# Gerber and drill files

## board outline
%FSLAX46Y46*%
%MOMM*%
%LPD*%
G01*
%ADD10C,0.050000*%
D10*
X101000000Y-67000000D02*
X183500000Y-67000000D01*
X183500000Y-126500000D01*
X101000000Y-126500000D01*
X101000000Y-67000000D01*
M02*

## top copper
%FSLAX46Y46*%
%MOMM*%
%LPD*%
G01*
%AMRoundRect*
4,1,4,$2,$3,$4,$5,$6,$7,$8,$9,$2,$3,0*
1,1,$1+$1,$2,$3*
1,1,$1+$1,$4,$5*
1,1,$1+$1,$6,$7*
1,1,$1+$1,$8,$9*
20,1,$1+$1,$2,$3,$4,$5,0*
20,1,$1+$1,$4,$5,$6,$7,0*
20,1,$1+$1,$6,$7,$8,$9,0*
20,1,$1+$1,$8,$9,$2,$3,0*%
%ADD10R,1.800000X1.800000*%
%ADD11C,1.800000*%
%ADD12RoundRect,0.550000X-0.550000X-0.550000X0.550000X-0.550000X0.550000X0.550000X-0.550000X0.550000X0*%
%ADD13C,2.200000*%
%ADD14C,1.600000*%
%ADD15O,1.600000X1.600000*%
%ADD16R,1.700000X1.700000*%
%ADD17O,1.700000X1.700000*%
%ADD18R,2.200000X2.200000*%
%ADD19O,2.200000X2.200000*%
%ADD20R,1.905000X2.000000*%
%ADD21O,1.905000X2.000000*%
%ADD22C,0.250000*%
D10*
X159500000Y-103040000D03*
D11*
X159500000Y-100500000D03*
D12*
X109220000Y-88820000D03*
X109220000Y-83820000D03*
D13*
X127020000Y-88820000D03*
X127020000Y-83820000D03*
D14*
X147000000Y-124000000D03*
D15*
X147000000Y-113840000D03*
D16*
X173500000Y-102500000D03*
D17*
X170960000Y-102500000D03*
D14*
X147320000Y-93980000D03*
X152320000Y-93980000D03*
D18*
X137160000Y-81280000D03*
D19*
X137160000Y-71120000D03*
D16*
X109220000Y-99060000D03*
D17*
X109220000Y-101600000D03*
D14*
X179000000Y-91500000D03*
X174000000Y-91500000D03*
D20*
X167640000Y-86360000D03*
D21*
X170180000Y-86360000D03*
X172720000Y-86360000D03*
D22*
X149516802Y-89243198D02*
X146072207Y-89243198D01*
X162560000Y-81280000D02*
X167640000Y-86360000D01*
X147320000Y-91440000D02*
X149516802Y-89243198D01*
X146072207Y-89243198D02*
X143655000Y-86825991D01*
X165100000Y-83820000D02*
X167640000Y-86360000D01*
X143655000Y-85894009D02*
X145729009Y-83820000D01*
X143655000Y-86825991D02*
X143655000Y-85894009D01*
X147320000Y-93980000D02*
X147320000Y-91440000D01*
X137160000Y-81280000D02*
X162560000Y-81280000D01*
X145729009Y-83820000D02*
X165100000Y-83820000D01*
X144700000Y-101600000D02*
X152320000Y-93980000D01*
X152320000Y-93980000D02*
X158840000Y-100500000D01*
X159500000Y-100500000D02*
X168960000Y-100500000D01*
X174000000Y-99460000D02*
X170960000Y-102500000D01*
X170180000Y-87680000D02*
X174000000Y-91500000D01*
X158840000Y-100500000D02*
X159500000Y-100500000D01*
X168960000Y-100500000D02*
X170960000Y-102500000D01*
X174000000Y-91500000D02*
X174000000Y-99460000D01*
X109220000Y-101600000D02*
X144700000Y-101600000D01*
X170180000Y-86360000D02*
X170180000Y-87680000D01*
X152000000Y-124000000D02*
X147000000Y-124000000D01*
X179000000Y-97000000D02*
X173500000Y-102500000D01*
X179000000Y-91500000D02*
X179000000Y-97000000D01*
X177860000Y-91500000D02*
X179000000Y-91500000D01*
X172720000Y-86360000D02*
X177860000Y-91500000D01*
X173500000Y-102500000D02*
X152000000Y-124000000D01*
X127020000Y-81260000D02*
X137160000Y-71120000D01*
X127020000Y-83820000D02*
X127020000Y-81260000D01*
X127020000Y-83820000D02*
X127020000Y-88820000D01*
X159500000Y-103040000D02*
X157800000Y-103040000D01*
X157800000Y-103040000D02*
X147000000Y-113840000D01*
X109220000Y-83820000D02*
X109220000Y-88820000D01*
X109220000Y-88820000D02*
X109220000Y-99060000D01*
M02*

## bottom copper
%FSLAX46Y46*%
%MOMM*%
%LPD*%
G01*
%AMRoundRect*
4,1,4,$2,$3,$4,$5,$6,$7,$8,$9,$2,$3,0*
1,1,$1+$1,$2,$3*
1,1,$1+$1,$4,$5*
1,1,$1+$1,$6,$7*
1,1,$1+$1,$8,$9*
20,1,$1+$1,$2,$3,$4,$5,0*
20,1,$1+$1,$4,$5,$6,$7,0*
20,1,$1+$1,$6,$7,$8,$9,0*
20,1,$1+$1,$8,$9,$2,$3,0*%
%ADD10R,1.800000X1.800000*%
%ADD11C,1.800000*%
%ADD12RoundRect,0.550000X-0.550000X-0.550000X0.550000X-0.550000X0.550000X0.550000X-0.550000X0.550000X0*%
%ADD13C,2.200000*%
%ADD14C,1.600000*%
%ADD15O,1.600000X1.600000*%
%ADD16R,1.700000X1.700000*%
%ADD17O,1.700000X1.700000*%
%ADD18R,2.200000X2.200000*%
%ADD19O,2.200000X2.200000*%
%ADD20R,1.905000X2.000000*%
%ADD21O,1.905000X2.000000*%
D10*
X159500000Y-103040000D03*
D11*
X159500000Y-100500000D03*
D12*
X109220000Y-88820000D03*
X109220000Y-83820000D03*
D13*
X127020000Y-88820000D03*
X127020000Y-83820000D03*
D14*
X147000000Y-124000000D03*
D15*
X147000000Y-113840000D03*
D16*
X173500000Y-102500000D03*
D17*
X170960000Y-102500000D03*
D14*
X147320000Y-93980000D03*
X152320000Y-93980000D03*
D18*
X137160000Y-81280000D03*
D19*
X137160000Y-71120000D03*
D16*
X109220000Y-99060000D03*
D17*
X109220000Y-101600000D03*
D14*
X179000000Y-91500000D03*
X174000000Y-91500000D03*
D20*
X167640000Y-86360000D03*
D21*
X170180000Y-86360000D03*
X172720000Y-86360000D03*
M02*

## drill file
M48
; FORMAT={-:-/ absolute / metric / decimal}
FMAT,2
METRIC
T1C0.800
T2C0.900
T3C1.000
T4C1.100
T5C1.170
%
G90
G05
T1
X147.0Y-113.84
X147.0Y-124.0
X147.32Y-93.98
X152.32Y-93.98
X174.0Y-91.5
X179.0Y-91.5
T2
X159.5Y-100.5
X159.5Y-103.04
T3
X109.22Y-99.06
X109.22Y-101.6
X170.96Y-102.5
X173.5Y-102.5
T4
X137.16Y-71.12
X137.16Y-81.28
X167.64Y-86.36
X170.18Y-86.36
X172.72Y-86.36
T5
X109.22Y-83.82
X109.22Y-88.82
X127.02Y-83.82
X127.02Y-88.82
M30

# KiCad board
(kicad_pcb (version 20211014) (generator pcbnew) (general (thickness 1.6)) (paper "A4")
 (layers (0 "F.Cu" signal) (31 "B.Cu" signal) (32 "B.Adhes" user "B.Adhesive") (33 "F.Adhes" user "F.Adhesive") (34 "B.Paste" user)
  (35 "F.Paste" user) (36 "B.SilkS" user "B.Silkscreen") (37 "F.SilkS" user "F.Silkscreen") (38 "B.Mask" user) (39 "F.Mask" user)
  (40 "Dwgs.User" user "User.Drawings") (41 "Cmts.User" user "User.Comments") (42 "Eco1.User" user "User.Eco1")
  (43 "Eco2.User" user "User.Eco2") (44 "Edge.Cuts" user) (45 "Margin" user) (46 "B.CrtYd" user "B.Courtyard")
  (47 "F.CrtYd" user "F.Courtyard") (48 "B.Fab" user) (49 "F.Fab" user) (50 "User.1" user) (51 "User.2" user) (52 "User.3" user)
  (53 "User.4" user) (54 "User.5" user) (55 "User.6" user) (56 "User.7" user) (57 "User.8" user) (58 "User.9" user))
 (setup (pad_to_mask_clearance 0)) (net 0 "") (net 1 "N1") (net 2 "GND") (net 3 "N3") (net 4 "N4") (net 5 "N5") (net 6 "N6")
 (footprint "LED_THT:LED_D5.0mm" (layer "F.Cu") (at 159.5 103.04 90)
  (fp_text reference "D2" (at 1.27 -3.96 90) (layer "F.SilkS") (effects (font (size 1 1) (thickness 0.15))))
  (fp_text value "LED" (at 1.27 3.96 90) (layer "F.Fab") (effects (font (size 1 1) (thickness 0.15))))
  (pad "1" thru_hole rect (at 0 0 90) (size 1.8 1.8) (drill 0.9) (layers *.Cu *.Mask) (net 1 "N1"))
  (pad "2" thru_hole circle (at 2.54 0 90) (size 1.8 1.8) (drill 0.9) (layers *.Cu *.Mask) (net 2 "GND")))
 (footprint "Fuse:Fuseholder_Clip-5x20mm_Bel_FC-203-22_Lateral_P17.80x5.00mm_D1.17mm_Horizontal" (layer "F.Cu") (at 109.22 83.82)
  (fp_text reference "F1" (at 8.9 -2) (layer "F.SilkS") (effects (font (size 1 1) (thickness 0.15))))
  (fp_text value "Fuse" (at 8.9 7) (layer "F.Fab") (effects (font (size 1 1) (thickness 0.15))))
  (pad "1" thru_hole roundrect (at 0 5) (size 2.2 2.2) (drill 1.17) (layers *.Cu *.Mask) (roundrect_rratio 0.25) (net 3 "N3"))
  (pad "1" thru_hole roundrect (at 0 0) (size 2.2 2.2) (drill 1.17) (layers *.Cu *.Mask) (roundrect_rratio 0.25) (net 3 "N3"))
  (pad "2" thru_hole circle (at 17.8 5) (size 2.2 2.2) (drill 1.17) (layers *.Cu *.Mask) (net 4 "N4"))
  (pad "2" thru_hole circle (at 17.8 0) (size 2.2 2.2) (drill 1.17) (layers *.Cu *.Mask) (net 4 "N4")))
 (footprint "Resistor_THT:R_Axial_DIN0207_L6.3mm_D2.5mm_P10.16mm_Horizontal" (layer "F.Cu") (at 147 124 90)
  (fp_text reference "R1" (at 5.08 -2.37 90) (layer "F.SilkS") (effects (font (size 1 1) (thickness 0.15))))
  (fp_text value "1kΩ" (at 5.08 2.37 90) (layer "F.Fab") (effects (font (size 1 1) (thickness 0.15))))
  (pad "1" thru_hole circle (at 0 0 90) (size 1.6 1.6) (drill 0.8) (layers *.Cu *.Mask) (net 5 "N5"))
  (pad "2" thru_hole oval (at 10.16 0 90) (size 1.6 1.6) (drill 0.8) (layers *.Cu *.Mask) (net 1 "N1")))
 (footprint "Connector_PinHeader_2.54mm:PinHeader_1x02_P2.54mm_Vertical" (layer "F.Cu") (at 173.5 102.5 -90)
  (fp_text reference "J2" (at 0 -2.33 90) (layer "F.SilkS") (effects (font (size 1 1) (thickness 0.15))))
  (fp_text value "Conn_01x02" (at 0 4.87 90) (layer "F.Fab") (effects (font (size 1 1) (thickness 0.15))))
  (pad "1" thru_hole rect (at 0 0 270) (size 1.7 1.7) (drill 1) (layers *.Cu *.Mask) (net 5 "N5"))
  (pad "2" thru_hole oval (at 0 2.54 270) (size 1.7 1.7) (drill 1) (layers *.Cu *.Mask) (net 2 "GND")))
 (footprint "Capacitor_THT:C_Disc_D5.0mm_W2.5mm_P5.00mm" (layer "F.Cu") (at 147.32 93.98)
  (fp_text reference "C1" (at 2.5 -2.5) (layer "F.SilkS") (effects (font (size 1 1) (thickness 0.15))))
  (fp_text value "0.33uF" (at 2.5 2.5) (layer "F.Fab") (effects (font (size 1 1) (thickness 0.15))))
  (pad "1" thru_hole circle (at 0 0) (size 1.6 1.6) (drill 0.8) (layers *.Cu *.Mask) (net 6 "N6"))
  (pad "2" thru_hole circle (at 5 0) (size 1.6 1.6) (drill 0.8) (layers *.Cu *.Mask) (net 2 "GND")))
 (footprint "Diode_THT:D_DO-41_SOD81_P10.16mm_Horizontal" (layer "F.Cu") (at 137.16 81.28 90)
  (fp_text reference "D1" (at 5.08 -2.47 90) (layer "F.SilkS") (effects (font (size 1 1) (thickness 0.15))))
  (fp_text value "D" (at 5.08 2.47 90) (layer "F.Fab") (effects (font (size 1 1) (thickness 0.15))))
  (pad "1" thru_hole rect (at 0 0 90) (size 2.2 2.2) (drill 1.1) (layers *.Cu *.Mask) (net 6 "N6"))
  (pad "2" thru_hole oval (at 10.16 0 90) (size 2.2 2.2) (drill 1.1) (layers *.Cu *.Mask) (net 4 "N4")))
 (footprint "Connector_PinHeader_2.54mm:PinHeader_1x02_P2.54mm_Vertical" (layer "F.Cu") (at 109.22 99.06)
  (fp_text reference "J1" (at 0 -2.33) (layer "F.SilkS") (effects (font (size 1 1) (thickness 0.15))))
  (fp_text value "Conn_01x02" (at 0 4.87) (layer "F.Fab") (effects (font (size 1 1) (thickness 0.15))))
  (pad "1" thru_hole rect (at 0 0) (size 1.7 1.7) (drill 1) (layers *.Cu *.Mask) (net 3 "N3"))
  (pad "2" thru_hole oval (at 0 2.54) (size 1.7 1.7) (drill 1) (layers *.Cu *.Mask) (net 2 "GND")))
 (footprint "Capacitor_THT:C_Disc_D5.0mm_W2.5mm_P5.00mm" (layer "B.Cu") (at 179 91.5 180)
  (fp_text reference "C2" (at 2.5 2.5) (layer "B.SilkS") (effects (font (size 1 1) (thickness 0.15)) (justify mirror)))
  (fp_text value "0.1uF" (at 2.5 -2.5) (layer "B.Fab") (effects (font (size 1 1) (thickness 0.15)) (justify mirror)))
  (pad "1" thru_hole circle (at 0 0 180) (size 1.6 1.6) (drill 0.8) (layers *.Cu *.Mask) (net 5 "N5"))
  (pad "2" thru_hole circle (at 5 0 180) (size 1.6 1.6) (drill 0.8) (layers *.Cu *.Mask) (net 2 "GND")))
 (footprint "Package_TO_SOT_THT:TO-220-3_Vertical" (layer "B.Cu") (at 167.64 86.36)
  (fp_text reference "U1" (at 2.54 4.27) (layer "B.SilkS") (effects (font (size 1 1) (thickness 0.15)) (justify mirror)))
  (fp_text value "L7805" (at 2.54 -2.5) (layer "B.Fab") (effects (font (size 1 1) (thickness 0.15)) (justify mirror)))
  (pad "1" thru_hole rect (at 0 0) (size 1.905 2) (drill 1.1) (layers *.Cu *.Mask) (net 6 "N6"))
  (pad "2" thru_hole oval (at 2.54 0) (size 1.905 2) (drill 1.1) (layers *.Cu *.Mask) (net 2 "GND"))
  (pad "3" thru_hole oval (at 5.08 0) (size 1.905 2) (drill 1.1) (layers *.Cu *.Mask) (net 5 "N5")))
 (gr_rect (start 101 67) (end 183.5 126.5) (layer "Edge.Cuts") (width 0.05) (fill none))
 (segment (start 149.516802 89.243198) (end 146.072207 89.243198) (width 0.25) (layer "F.Cu") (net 6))
 (segment (start 162.56 81.28) (end 167.64 86.36) (width 0.25) (layer "F.Cu") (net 6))
 (segment (start 147.32 91.44) (end 149.516802 89.243198) (width 0.25) (layer "F.Cu") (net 6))
 (segment (start 146.072207 89.243198) (end 143.655 86.825991) (width 0.25) (layer "F.Cu") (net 6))
 (segment (start 165.1 83.82) (end 167.64 86.36) (width 0.25) (layer "F.Cu") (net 6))
 (segment (start 143.655 85.894009) (end 145.729009 83.82) (width 0.25) (layer "F.Cu") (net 6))
 (segment (start 143.655 86.825991) (end 143.655 85.894009) (width 0.25) (layer "F.Cu") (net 6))
 (segment (start 147.32 93.98) (end 147.32 91.44) (width 0.25) (layer "F.Cu") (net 6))
 (segment (start 137.16 81.28) (end 162.56 81.28) (width 0.25) (layer "F.Cu") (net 6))
 (segment (start 145.729009 83.82) (end 165.1 83.82) (width 0.25) (layer "F.Cu") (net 6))
 (segment (start 144.7 101.6) (end 152.32 93.98) (width 0.25) (layer "F.Cu") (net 2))
 (segment (start 152.32 93.98) (end 158.84 100.5) (width 0.25) (layer "F.Cu") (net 2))
 (segment (start 159.5 100.5) (end 168.96 100.5) (width 0.25) (layer "F.Cu") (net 2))
 (segment (start 174 99.46) (end 170.96 102.5) (width 0.25) (layer "F.Cu") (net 2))
 (segment (start 170.18 87.68) (end 174 91.5) (width 0.25) (layer "F.Cu") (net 2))
 (segment (start 158.84 100.5) (end 159.5 100.5) (width 0.25) (layer "F.Cu") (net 2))
 (segment (start 168.96 100.5) (end 170.96 102.5) (width 0.25) (layer "F.Cu") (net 2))
 (segment (start 174 91.5) (end 174 99.46) (width 0.25) (layer "F.Cu") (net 2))
 (segment (start 109.22 101.6) (end 144.7 101.6) (width 0.25) (layer "F.Cu") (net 2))
 (segment (start 170.18 86.36) (end 170.18 87.68) (width 0.25) (layer "F.Cu") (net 2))
 (segment (start 152 124) (end 147 124) (width 0.25) (layer "F.Cu") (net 5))
 (segment (start 179 97) (end 173.5 102.5) (width 0.25) (layer "F.Cu") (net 5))
 (segment (start 179 91.5) (end 179 97) (width 0.25) (layer "F.Cu") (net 5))
 (segment (start 177.86 91.5) (end 179 91.5) (width 0.25) (layer "F.Cu") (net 5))
 (segment (start 172.72 86.36) (end 177.86 91.5) (width 0.25) (layer "F.Cu") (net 5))
 (segment (start 173.5 102.5) (end 152 124) (width 0.25) (layer "F.Cu") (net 5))
 (segment (start 127.02 81.26) (end 137.16 71.12) (width 0.25) (layer "F.Cu") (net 4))
 (segment (start 127.02 83.82) (end 127.02 81.26) (width 0.25) (layer "F.Cu") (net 4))
 (segment (start 127.02 83.82) (end 127.02 88.82) (width 0.25) (layer "F.Cu") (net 4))
 (segment (start 159.5 103.04) (end 157.8 103.04) (width 0.25) (layer "F.Cu") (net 1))
 (segment (start 157.8 103.04) (end 147 113.84) (width 0.25) (layer "F.Cu") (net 1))
 (segment (start 109.22 83.82) (end 109.22 88.82) (width 0.25) (layer "F.Cu") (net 3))
 (segment (start 109.22 88.82) (end 109.22 99.06) (width 0.25) (layer "F.Cu") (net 3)))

